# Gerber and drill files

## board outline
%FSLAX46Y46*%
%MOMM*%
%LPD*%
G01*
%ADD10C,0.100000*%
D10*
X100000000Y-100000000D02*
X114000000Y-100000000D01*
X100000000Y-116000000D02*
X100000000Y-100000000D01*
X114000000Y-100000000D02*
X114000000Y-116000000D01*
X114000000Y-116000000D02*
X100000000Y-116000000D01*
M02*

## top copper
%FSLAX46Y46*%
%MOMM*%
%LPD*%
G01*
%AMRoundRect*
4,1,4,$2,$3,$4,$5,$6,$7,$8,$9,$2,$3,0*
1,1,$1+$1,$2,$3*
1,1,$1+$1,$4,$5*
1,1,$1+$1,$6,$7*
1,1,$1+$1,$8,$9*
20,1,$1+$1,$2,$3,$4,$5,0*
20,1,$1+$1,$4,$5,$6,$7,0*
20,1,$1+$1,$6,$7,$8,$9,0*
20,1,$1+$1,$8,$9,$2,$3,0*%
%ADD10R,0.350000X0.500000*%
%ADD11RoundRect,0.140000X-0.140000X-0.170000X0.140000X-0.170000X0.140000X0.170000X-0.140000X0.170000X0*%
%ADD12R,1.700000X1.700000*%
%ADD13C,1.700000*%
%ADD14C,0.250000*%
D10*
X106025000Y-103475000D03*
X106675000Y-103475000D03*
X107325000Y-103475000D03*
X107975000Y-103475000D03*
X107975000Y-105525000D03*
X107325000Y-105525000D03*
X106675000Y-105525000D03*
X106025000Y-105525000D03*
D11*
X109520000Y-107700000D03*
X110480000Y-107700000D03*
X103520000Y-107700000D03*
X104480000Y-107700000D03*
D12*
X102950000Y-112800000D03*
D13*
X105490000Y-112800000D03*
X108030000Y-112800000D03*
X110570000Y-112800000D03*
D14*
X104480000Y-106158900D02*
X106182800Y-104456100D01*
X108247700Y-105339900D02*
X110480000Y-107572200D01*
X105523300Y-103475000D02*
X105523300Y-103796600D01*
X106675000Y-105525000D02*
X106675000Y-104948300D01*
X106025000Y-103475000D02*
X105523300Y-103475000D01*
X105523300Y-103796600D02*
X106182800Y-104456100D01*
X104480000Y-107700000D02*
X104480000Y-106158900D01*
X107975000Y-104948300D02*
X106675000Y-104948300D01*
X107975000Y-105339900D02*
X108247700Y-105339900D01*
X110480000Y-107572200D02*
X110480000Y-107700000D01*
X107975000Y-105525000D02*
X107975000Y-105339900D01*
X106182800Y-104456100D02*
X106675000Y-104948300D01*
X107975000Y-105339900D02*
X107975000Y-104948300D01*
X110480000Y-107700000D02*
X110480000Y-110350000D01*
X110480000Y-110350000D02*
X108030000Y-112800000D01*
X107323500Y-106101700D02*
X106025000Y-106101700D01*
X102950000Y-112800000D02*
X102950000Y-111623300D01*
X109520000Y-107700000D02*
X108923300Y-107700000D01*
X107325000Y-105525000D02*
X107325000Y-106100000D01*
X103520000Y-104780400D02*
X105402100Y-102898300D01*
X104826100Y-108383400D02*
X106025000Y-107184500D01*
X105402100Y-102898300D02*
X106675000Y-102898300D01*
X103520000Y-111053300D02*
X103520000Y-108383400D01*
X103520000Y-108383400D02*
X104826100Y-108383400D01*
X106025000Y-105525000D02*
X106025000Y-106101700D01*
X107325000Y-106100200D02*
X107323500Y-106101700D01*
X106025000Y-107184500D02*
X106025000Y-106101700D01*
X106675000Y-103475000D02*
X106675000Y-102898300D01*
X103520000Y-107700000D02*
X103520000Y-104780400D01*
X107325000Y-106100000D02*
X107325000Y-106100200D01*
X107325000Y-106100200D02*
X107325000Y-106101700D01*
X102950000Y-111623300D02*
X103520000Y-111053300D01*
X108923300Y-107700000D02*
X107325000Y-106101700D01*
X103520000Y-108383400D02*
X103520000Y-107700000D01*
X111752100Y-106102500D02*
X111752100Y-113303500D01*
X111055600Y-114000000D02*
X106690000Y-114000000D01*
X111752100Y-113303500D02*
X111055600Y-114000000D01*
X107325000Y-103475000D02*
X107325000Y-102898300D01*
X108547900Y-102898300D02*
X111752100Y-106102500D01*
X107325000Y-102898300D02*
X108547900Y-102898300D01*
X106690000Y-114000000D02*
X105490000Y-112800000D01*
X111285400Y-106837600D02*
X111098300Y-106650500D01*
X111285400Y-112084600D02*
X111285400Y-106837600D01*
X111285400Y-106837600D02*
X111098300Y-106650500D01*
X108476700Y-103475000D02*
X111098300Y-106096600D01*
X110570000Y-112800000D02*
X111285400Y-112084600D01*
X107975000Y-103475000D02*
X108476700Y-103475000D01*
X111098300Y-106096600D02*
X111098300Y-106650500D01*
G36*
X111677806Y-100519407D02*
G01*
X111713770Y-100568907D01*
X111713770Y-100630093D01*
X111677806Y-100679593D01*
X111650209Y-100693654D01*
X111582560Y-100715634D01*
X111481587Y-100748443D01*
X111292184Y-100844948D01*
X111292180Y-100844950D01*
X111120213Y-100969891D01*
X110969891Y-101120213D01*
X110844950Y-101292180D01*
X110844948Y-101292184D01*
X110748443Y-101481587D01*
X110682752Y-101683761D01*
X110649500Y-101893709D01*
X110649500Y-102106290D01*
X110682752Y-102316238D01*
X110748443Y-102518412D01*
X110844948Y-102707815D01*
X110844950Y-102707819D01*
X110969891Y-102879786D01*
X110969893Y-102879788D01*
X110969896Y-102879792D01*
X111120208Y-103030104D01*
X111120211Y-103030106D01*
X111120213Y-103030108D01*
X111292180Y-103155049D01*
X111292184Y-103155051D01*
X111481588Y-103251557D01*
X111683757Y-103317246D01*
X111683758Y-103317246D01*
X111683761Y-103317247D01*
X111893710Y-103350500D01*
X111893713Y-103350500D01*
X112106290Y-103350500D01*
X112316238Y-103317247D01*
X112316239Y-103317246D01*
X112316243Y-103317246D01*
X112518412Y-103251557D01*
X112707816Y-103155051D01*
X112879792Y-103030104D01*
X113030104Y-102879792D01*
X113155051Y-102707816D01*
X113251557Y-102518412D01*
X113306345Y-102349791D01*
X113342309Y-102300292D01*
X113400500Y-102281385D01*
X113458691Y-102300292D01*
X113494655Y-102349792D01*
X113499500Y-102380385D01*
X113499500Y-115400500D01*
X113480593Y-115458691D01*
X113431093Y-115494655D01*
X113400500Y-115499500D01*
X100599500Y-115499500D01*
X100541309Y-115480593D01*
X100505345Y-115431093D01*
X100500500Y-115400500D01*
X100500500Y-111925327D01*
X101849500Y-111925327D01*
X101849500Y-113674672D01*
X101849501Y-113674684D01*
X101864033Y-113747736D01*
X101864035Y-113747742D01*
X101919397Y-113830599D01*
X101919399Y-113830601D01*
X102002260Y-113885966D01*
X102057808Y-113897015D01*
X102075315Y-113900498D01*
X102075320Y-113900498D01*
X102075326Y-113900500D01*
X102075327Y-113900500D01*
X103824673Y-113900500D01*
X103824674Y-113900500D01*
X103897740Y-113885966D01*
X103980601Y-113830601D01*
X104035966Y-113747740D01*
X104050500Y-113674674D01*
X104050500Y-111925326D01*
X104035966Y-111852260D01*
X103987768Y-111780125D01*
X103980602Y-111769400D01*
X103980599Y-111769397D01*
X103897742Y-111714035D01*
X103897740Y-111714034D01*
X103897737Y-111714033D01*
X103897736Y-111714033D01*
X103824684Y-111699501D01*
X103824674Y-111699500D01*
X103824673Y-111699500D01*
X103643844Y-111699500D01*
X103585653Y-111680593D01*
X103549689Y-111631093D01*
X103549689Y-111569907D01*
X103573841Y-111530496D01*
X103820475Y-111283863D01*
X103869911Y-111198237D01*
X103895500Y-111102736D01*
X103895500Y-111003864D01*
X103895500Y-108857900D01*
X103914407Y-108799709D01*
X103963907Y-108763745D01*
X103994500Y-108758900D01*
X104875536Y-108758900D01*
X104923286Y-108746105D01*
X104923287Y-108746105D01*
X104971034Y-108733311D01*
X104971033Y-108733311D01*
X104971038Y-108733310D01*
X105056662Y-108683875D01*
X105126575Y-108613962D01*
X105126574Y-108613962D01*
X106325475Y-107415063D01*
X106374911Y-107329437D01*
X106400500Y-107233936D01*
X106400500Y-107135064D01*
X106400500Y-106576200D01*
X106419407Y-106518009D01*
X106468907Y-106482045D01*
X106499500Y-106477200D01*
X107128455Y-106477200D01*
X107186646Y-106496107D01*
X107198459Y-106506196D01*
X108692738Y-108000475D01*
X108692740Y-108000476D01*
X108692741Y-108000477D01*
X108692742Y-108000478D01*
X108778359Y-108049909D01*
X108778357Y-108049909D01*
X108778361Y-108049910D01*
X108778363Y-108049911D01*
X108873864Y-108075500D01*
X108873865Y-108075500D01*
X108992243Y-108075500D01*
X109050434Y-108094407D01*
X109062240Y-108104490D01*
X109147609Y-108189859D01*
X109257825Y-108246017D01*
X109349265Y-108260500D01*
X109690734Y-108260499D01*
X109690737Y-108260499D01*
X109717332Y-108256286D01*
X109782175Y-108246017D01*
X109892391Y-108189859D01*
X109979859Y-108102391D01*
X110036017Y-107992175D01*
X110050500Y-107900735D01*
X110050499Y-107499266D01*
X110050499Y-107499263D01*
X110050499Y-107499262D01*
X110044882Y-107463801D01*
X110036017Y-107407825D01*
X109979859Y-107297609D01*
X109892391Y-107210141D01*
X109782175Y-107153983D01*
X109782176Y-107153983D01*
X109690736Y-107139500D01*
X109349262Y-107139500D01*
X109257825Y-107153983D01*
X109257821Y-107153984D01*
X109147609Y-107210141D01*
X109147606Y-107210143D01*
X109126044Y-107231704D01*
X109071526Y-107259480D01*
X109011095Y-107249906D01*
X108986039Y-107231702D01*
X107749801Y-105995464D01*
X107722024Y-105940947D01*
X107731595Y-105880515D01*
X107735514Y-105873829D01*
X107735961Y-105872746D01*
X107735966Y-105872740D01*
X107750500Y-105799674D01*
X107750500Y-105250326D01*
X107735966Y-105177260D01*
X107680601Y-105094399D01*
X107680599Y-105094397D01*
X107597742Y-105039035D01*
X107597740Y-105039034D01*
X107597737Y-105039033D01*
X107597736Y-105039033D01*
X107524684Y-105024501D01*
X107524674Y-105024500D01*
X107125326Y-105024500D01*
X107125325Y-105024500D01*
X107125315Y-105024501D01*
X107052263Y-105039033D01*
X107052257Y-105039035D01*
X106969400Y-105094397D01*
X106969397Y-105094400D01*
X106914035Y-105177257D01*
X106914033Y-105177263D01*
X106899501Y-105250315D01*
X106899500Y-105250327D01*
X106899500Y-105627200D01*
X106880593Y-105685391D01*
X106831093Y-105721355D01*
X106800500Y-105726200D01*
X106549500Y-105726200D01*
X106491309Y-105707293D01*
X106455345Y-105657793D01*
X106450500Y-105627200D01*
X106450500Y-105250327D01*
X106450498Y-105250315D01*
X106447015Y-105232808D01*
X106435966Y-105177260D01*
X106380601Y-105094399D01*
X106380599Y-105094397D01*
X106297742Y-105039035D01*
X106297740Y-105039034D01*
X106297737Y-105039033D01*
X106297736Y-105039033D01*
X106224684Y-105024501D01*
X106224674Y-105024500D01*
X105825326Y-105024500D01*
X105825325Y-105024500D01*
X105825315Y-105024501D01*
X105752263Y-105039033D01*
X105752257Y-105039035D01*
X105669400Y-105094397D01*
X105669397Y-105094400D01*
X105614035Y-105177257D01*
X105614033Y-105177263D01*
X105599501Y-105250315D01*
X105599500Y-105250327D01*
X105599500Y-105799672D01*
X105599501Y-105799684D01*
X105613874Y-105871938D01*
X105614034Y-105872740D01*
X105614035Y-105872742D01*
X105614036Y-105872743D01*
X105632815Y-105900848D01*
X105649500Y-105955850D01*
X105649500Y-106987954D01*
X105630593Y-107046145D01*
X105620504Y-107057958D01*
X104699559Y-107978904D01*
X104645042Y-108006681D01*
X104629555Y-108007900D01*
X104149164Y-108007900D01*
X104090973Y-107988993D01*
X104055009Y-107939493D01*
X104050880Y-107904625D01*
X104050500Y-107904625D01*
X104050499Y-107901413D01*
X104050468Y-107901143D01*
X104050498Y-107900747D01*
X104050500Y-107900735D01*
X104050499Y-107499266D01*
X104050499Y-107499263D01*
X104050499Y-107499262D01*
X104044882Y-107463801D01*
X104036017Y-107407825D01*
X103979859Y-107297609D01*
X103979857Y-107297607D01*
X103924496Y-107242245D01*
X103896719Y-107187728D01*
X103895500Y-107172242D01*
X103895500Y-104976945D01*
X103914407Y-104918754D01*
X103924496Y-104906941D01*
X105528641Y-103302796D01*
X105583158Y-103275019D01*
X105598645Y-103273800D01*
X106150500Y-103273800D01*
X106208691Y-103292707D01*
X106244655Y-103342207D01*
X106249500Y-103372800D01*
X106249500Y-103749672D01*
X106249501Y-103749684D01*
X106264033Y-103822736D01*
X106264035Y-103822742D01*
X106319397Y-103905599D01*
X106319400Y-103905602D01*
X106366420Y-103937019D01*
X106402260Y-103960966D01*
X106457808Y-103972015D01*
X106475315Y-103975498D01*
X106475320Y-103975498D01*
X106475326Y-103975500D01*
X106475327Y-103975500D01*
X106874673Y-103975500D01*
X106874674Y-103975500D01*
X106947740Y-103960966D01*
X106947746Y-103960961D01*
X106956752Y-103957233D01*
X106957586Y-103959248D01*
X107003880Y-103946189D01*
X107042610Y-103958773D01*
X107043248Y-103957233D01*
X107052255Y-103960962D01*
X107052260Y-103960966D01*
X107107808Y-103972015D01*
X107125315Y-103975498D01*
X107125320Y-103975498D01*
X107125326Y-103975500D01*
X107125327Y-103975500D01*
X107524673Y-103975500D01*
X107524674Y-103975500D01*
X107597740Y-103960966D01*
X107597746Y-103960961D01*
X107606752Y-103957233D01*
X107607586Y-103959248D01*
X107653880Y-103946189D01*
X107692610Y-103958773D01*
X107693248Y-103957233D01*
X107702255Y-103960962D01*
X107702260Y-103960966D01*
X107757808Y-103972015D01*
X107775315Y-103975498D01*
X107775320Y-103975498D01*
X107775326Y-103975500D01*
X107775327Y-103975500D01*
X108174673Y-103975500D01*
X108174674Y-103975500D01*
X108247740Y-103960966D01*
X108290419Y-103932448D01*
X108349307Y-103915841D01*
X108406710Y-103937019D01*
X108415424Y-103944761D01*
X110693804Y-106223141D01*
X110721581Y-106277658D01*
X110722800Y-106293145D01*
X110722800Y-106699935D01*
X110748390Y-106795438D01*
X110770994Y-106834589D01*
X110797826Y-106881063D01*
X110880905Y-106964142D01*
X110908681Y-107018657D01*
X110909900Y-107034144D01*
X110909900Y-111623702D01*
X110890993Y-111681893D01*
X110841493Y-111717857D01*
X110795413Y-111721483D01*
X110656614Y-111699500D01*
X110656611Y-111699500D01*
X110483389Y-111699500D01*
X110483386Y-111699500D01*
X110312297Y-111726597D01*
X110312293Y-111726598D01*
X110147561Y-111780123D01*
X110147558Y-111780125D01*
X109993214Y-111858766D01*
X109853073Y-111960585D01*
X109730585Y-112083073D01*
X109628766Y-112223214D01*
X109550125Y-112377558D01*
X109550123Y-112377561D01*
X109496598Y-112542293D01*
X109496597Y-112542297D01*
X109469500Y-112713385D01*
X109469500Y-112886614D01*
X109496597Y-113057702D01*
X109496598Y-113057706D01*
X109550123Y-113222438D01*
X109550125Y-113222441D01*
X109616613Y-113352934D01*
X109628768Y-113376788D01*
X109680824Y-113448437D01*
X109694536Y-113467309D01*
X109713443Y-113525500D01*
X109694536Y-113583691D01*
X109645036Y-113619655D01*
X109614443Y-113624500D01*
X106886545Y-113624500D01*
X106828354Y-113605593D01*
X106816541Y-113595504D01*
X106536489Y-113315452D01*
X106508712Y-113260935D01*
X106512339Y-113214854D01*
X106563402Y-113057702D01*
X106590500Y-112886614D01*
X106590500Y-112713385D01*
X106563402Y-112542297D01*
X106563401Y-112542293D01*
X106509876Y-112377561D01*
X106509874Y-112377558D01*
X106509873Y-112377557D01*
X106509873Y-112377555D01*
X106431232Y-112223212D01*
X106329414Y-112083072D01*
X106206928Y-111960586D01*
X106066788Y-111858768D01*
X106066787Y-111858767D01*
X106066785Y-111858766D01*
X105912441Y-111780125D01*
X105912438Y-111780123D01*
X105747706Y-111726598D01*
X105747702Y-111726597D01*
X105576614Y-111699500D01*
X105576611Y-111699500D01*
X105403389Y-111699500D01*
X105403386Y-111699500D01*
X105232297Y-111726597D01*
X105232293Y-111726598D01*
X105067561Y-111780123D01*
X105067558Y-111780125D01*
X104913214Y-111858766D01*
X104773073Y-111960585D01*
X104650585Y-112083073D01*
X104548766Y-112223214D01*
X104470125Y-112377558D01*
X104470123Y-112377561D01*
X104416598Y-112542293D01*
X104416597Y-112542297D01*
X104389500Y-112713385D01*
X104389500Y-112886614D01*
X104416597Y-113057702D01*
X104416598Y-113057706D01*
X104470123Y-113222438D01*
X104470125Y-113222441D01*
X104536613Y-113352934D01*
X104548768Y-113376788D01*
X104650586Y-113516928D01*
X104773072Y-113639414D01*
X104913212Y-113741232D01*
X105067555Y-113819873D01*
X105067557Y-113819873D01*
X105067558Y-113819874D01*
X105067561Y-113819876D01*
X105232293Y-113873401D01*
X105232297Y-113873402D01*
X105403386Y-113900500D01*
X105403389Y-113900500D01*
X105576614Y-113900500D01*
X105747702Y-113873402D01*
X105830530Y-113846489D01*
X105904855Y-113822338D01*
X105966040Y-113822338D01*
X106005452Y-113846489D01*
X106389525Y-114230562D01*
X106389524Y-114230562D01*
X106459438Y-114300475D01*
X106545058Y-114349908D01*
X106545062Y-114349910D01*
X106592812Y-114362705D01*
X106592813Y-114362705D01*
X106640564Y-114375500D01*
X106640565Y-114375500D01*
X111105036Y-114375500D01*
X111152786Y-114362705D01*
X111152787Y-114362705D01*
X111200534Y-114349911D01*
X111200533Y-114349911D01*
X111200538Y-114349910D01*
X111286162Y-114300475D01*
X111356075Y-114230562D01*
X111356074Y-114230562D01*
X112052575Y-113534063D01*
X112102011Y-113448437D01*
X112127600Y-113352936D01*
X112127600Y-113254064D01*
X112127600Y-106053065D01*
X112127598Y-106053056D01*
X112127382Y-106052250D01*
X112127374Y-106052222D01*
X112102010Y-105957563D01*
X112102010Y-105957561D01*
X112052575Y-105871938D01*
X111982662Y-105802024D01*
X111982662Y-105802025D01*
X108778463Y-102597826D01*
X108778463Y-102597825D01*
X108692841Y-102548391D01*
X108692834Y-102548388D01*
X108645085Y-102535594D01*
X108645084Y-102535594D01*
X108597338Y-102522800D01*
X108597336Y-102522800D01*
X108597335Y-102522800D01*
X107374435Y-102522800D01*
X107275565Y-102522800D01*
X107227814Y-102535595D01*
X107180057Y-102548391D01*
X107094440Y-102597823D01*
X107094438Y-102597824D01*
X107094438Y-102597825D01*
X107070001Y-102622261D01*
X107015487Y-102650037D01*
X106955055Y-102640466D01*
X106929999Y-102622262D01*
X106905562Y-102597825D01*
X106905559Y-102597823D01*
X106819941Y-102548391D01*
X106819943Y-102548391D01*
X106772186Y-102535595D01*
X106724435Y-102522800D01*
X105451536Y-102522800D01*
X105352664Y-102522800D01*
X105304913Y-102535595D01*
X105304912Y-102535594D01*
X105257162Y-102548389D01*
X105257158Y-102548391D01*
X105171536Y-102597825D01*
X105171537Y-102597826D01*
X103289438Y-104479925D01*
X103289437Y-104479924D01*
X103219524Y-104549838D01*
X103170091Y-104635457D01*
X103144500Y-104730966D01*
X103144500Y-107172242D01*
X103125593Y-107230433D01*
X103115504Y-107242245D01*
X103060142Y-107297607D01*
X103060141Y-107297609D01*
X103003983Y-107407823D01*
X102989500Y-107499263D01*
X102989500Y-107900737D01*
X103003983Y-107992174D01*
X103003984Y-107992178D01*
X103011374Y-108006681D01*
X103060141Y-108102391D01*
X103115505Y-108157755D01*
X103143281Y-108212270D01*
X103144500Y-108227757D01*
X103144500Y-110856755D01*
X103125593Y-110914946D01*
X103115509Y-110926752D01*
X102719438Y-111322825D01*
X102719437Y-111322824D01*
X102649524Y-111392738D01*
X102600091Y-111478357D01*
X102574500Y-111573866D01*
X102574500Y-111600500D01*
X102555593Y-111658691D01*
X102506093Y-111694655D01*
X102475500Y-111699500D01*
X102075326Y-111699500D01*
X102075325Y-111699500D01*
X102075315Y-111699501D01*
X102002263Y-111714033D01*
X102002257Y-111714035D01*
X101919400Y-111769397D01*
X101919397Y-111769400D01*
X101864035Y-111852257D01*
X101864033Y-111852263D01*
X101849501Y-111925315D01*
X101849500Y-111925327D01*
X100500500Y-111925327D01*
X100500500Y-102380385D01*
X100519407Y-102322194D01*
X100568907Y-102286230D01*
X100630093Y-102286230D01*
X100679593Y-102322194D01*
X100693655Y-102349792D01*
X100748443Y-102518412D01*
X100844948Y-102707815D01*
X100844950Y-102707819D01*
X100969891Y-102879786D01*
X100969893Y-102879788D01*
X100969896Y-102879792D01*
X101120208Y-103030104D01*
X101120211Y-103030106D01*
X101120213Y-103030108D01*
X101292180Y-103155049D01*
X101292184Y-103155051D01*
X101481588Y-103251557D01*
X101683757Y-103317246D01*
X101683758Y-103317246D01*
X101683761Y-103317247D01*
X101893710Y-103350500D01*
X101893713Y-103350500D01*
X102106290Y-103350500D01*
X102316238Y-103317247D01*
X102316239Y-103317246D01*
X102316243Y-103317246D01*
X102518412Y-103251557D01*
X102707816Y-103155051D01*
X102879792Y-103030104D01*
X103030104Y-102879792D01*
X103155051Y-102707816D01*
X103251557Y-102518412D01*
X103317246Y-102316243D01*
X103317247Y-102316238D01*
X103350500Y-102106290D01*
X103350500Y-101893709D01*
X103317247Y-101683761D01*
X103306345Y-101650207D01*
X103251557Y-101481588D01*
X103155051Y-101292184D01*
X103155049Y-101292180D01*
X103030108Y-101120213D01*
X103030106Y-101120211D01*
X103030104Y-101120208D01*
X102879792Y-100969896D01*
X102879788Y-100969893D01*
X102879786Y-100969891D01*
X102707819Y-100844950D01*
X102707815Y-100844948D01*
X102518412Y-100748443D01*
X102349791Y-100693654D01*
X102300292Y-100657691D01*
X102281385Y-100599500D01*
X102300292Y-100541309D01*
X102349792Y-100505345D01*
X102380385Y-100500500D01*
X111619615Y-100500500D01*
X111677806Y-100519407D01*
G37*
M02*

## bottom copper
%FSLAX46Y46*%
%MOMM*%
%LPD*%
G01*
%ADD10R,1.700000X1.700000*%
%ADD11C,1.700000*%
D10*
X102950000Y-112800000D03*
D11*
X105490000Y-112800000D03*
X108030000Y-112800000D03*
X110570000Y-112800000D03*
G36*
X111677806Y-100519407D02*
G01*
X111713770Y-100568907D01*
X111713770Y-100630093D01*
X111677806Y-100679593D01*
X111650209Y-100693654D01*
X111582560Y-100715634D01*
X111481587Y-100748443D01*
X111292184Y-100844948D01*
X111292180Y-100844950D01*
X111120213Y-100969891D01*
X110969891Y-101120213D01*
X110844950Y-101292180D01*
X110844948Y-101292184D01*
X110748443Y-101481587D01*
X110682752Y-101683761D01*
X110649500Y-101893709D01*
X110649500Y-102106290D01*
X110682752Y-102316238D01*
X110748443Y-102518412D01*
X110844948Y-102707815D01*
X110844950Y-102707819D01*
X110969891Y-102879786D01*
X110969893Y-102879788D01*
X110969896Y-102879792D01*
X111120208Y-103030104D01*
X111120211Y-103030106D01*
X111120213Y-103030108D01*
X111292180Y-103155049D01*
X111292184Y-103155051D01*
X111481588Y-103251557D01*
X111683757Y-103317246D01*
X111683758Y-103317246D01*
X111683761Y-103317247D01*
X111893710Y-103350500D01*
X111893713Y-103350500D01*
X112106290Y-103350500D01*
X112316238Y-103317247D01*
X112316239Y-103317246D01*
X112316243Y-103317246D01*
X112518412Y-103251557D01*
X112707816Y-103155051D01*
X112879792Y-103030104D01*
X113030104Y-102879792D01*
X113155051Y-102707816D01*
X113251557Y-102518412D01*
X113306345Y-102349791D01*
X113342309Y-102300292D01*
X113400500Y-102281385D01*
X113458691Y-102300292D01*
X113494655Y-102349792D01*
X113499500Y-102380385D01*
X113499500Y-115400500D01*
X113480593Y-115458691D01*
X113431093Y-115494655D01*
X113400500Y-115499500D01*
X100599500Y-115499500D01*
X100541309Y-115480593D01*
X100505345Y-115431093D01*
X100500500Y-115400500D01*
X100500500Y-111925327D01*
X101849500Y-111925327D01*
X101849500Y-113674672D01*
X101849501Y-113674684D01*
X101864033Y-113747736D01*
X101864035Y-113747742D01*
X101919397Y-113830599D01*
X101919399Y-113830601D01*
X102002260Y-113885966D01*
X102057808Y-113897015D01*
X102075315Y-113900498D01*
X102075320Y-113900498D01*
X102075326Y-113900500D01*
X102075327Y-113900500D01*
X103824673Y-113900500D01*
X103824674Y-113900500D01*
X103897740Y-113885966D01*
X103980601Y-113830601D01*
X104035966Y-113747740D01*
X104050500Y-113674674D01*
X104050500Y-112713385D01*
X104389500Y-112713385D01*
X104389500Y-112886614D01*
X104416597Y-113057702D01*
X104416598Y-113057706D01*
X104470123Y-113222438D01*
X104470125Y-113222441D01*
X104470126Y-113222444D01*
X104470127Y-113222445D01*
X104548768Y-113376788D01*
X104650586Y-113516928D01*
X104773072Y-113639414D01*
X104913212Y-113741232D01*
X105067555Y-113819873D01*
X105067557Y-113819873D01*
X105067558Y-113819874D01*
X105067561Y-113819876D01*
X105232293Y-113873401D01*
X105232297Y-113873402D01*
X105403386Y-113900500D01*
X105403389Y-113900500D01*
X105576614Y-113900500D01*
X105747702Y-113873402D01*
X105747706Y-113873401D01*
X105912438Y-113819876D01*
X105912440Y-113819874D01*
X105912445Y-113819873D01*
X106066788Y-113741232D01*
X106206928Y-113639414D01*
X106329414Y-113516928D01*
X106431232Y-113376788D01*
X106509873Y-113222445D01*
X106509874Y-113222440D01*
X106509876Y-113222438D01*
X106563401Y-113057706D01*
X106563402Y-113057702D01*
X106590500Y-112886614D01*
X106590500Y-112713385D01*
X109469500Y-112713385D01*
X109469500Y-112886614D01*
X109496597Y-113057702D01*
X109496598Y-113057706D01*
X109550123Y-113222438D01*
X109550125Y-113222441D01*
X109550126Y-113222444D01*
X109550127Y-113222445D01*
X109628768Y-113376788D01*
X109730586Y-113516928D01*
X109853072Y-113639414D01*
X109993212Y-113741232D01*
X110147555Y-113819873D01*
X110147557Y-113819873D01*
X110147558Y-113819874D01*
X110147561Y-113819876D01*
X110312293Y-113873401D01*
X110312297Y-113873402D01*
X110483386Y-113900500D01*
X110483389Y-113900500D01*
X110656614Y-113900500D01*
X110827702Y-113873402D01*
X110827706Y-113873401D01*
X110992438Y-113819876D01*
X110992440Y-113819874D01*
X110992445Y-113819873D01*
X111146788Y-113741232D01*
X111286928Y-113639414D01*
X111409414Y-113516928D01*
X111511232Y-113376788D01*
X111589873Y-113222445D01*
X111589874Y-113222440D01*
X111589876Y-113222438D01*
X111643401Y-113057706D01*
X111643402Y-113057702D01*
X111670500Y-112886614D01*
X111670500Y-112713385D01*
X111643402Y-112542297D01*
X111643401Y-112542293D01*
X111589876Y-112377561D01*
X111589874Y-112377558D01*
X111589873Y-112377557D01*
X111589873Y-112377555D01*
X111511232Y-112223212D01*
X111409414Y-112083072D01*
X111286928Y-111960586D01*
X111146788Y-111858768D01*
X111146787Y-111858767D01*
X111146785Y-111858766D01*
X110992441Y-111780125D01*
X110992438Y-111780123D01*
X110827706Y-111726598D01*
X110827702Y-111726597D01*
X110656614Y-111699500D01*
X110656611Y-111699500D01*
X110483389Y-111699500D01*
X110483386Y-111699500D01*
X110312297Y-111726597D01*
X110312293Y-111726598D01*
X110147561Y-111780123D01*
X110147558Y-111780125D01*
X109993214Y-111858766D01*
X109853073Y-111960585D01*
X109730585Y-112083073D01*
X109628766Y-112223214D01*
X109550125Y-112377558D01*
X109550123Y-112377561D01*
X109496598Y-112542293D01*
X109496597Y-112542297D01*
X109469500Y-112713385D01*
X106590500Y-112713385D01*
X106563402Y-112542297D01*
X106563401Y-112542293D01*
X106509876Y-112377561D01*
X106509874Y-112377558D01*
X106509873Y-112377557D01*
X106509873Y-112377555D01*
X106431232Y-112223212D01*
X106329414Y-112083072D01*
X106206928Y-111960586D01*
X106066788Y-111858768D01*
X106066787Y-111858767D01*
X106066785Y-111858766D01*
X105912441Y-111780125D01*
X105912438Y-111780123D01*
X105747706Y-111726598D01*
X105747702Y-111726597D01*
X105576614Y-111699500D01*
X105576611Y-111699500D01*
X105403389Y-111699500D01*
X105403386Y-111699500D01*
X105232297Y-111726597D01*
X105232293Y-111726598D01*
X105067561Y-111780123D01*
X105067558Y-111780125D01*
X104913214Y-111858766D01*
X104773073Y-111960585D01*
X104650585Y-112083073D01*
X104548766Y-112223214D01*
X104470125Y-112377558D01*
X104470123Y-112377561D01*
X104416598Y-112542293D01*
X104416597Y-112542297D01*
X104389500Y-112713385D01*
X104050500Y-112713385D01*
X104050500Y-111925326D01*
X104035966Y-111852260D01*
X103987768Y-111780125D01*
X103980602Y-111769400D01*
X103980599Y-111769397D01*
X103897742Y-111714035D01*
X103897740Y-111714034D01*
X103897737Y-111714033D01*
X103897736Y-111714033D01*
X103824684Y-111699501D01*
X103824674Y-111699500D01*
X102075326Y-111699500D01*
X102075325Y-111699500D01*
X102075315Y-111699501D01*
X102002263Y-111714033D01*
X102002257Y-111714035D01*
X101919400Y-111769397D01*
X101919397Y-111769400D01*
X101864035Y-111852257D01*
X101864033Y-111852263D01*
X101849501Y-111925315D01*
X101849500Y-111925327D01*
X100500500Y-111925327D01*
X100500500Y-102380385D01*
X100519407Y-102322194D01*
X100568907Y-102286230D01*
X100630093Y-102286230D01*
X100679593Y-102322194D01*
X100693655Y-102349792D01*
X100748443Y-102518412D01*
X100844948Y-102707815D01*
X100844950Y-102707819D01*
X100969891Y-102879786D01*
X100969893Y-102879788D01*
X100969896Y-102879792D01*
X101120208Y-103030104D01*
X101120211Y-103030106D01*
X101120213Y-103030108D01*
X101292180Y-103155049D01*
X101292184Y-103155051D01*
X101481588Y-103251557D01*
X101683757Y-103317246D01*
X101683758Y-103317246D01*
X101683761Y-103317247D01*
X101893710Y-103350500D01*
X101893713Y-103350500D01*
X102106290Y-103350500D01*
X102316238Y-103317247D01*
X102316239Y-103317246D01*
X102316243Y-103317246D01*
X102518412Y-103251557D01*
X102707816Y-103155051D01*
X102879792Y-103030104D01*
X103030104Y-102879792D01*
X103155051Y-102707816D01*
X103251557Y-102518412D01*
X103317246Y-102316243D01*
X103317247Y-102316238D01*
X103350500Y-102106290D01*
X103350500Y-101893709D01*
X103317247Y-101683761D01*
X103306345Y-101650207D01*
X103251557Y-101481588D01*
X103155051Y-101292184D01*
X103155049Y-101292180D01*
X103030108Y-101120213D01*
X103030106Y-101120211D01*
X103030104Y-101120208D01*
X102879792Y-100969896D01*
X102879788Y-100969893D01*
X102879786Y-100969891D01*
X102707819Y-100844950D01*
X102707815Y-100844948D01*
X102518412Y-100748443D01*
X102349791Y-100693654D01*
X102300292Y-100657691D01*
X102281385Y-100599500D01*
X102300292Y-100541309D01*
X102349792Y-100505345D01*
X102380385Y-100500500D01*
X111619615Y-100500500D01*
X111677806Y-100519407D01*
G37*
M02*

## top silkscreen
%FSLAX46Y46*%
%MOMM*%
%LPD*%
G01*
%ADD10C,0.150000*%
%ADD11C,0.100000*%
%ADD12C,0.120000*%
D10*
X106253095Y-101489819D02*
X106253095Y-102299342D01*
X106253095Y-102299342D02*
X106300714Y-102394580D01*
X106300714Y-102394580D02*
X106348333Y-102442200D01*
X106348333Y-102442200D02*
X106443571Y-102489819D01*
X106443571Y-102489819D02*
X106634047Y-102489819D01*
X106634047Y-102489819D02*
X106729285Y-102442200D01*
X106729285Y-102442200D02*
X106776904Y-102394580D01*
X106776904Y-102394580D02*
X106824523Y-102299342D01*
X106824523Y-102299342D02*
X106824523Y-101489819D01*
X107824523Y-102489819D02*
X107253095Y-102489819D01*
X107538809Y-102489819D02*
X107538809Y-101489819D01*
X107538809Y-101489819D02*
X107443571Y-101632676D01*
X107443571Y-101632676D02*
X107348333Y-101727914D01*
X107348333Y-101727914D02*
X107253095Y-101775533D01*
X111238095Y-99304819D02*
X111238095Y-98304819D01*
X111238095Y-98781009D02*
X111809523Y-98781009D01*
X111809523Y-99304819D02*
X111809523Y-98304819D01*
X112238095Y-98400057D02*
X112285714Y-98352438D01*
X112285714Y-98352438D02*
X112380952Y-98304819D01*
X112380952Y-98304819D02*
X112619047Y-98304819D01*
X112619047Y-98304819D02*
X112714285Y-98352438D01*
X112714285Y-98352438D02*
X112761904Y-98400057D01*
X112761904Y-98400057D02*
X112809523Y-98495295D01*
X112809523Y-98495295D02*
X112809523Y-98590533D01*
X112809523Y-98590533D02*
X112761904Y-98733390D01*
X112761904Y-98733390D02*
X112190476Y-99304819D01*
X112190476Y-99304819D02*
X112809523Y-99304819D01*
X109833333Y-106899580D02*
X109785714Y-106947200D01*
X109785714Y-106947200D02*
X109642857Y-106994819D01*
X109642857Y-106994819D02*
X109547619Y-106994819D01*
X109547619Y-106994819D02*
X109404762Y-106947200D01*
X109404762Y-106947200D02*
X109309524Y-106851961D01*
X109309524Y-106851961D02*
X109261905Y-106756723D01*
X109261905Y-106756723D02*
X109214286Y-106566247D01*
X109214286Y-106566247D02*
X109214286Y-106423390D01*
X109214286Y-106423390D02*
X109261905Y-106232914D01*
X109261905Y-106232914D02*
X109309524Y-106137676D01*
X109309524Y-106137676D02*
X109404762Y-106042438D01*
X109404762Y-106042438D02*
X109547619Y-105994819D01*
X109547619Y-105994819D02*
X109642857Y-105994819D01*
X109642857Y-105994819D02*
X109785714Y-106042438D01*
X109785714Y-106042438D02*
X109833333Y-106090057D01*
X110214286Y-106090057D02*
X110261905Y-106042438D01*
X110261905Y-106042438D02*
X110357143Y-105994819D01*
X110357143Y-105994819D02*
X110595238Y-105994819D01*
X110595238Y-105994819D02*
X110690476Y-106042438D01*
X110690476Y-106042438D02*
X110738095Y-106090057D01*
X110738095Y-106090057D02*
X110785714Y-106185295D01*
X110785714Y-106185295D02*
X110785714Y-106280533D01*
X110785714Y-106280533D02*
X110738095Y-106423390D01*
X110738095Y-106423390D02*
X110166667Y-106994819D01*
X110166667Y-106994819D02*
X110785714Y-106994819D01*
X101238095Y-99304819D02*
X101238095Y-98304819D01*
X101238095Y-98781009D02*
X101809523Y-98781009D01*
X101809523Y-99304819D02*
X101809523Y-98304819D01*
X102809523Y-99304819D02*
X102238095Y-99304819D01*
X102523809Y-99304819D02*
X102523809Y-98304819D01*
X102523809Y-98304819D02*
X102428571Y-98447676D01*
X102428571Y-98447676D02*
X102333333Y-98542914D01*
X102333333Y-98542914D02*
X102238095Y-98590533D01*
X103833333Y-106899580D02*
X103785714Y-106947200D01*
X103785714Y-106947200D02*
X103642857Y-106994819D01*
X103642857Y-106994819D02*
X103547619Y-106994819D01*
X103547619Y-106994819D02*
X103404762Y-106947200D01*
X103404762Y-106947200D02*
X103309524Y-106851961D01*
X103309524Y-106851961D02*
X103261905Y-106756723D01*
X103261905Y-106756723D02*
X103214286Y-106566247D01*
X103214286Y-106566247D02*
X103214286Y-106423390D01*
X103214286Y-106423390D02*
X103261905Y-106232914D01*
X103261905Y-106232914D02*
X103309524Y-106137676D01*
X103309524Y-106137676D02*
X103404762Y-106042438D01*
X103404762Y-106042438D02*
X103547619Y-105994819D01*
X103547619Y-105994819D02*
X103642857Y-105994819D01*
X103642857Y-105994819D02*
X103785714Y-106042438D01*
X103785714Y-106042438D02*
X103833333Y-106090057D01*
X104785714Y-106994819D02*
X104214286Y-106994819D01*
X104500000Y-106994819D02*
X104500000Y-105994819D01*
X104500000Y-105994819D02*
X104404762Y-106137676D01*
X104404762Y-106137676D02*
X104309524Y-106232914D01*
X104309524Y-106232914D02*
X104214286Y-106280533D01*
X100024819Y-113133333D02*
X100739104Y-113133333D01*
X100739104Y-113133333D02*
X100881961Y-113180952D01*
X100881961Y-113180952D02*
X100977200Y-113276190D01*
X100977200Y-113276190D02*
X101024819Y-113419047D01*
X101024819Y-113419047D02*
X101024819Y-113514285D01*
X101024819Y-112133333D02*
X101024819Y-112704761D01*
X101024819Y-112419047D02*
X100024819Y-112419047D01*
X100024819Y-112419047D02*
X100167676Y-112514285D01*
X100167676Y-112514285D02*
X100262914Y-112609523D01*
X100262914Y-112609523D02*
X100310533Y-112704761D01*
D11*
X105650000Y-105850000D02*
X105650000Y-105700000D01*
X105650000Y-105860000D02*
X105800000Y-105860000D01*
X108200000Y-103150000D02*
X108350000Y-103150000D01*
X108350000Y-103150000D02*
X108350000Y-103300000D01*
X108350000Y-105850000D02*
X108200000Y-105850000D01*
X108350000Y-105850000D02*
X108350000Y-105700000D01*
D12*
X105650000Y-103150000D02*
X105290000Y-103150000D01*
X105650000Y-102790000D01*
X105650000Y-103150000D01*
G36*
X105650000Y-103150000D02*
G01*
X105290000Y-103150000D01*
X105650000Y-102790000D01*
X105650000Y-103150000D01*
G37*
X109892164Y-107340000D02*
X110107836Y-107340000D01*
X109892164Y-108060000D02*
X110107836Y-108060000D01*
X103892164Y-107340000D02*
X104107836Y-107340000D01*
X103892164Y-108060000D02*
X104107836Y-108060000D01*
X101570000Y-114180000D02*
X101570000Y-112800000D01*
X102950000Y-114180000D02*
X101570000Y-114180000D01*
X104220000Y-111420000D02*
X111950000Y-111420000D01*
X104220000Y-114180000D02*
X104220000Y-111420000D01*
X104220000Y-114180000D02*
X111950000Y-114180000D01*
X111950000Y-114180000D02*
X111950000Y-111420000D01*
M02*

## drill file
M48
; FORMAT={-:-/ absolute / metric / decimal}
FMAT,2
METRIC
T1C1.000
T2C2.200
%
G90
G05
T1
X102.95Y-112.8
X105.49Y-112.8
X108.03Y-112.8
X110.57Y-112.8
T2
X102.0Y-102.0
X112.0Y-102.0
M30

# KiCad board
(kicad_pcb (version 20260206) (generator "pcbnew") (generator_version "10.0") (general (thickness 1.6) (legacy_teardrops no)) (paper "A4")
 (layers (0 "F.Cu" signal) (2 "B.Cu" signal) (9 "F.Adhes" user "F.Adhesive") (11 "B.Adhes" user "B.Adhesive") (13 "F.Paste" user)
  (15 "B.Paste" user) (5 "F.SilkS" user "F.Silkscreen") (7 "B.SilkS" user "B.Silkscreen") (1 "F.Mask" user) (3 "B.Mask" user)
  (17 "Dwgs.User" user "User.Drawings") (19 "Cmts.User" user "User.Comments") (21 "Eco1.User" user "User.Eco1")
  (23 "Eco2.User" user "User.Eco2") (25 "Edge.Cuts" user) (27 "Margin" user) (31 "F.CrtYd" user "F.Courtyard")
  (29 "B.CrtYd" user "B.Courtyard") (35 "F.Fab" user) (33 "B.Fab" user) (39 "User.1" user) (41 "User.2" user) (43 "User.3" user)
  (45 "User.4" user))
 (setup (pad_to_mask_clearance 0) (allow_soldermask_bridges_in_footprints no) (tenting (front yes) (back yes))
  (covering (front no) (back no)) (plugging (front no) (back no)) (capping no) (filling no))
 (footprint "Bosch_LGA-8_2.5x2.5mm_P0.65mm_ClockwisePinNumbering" (layer "F.Cu") (at 107 104.5)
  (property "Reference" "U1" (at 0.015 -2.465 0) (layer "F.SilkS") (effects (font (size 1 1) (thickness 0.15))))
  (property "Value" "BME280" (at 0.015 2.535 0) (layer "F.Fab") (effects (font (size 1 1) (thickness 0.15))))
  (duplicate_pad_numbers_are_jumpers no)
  (fp_line (start -1.35 1.35) (end -1.35 1.2) (stroke (width 0.1) (type solid)) (layer "F.SilkS"))
  (fp_line (start -1.35 1.36) (end -1.2 1.36) (stroke (width 0.1) (type solid)) (layer "F.SilkS"))
  (fp_line (start 1.2 -1.35) (end 1.35 -1.35) (stroke (width 0.1) (type solid)) (layer "F.SilkS"))
  (fp_line (start 1.35 -1.35) (end 1.35 -1.2) (stroke (width 0.1) (type solid)) (layer "F.SilkS"))
  (fp_line (start 1.35 1.35) (end 1.2 1.35) (stroke (width 0.1) (type solid)) (layer "F.SilkS"))
  (fp_line (start 1.35 1.35) (end 1.35 1.2) (stroke (width 0.1) (type solid)) (layer "F.SilkS"))
  (fp_poly
   (pts (xy -1.35 -1.35) (xy -1.71 -1.35) (xy -1.35 -1.71) (xy -1.35 -1.35)) (stroke (width 0.12) (type solid)) (fill yes) (layer "F.SilkS"))
  (pad "1" smd rect (at -0.975 -1.025 90) (size 0.5 0.35) (layers "F.Cu" "F.Mask" "F.Paste") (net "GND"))
  (pad "2" smd rect (at -0.325 -1.025 90) (size 0.5 0.35) (layers "F.Cu" "F.Mask" "F.Paste") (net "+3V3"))
  (pad "3" smd rect (at 0.325 -1.025 90) (size 0.5 0.35) (layers "F.Cu" "F.Mask" "F.Paste") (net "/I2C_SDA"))
  (pad "4" smd rect (at 0.975 -1.025 90) (size 0.5 0.35) (layers "F.Cu" "F.Mask" "F.Paste") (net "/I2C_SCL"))
  (pad "5" smd rect (at 0.975 1.025 90) (size 0.5 0.35) (layers "F.Cu" "F.Mask" "F.Paste") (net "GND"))
  (pad "6" smd rect (at 0.325 1.025 90) (size 0.5 0.35) (layers "F.Cu" "F.Mask" "F.Paste") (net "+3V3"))
  (pad "7" smd rect (at -0.325 1.025 90) (size 0.5 0.35) (layers "F.Cu" "F.Mask" "F.Paste") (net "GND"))
  (pad "8" smd rect (at -0.975 1.025 90) (size 0.5 0.35) (layers "F.Cu" "F.Mask" "F.Paste") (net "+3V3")))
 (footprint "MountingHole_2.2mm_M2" (layer "F.Cu") (at 112 102)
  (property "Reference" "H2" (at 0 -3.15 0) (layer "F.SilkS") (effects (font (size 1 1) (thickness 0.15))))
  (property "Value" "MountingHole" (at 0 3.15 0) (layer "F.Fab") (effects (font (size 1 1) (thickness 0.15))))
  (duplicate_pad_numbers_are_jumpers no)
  (pad "" np_thru_hole circle (at 0 0) (size 2.2 2.2) (drill 2.2) (layers "*.Cu" "*.Mask")))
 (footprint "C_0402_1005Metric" (layer "F.Cu") (at 110 107.7)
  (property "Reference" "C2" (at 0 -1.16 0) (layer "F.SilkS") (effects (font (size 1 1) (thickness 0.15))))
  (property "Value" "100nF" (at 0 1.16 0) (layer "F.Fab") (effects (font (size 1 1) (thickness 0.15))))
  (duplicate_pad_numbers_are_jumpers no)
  (fp_line (start -0.107836 -0.36) (end 0.107836 -0.36) (stroke (width 0.12) (type solid)) (layer "F.SilkS"))
  (fp_line (start -0.107836 0.36) (end 0.107836 0.36) (stroke (width 0.12) (type solid)) (layer "F.SilkS"))
  (pad "1" smd roundrect (at -0.48 0) (size 0.56 0.62) (layers "F.Cu" "F.Mask" "F.Paste") (roundrect_rratio 0.25) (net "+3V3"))
  (pad "2" smd roundrect (at 0.48 0) (size 0.56 0.62) (layers "F.Cu" "F.Mask" "F.Paste") (roundrect_rratio 0.25) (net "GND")))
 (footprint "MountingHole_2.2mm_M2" (layer "F.Cu") (at 102 102)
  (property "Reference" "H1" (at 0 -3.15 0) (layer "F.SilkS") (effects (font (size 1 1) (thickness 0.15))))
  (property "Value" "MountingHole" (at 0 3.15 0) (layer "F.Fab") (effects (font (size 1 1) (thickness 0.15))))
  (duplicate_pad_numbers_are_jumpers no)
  (pad "" np_thru_hole circle (at 0 0) (size 2.2 2.2) (drill 2.2) (layers "*.Cu" "*.Mask")))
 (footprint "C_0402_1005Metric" (layer "F.Cu") (at 104 107.7)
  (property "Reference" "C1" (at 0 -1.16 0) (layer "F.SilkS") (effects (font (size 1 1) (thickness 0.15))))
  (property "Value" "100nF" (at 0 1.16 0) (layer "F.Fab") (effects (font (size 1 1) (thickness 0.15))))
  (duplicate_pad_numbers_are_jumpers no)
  (fp_line (start -0.107836 -0.36) (end 0.107836 -0.36) (stroke (width 0.12) (type solid)) (layer "F.SilkS"))
  (fp_line (start -0.107836 0.36) (end 0.107836 0.36) (stroke (width 0.12) (type solid)) (layer "F.SilkS"))
  (pad "1" smd roundrect (at -0.48 0) (size 0.56 0.62) (layers "F.Cu" "F.Mask" "F.Paste") (roundrect_rratio 0.25) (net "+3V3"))
  (pad "2" smd roundrect (at 0.48 0) (size 0.56 0.62) (layers "F.Cu" "F.Mask" "F.Paste") (roundrect_rratio 0.25) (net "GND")))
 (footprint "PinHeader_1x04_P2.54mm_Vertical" (layer "F.Cu") (at 102.95 112.8 90)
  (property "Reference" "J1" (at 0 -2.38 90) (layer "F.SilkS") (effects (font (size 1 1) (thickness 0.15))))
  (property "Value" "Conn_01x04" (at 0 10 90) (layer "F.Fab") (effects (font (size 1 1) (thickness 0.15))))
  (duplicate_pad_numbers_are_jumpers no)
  (fp_line (start -1.38 -1.38) (end 0 -1.38) (stroke (width 0.12) (type solid)) (layer "F.SilkS"))
  (fp_line (start -1.38 0) (end -1.38 -1.38) (stroke (width 0.12) (type solid)) (layer "F.SilkS"))
  (fp_line (start 1.38 1.27) (end 1.38 9) (stroke (width 0.12) (type solid)) (layer "F.SilkS"))
  (fp_line (start -1.38 1.27) (end 1.38 1.27) (stroke (width 0.12) (type solid)) (layer "F.SilkS"))
  (fp_line (start -1.38 1.27) (end -1.38 9) (stroke (width 0.12) (type solid)) (layer "F.SilkS"))
  (fp_line (start -1.38 9) (end 1.38 9) (stroke (width 0.12) (type solid)) (layer "F.SilkS"))
  (pad "1" thru_hole rect (at 0 0 90) (size 1.7 1.7) (drill 1) (layers "*.Cu" "*.Mask") (remove_unused_layers no) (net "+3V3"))
  (pad "2" thru_hole circle (at 0 2.54 90) (size 1.7 1.7) (drill 1) (layers "*.Cu" "*.Mask") (remove_unused_layers no) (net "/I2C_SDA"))
  (pad "3" thru_hole circle (at 0 5.08 90) (size 1.7 1.7) (drill 1) (layers "*.Cu" "*.Mask") (remove_unused_layers no) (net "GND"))
  (pad "4" thru_hole circle (at 0 7.62 90) (size 1.7 1.7) (drill 1) (layers "*.Cu" "*.Mask") (remove_unused_layers no) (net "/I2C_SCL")))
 (gr_line (start 100 100) (end 114 100) (stroke (width 0.1) (type default)) (layer "Edge.Cuts"))
 (gr_line (start 100 116) (end 100 100) (stroke (width 0.1) (type default)) (layer "Edge.Cuts"))
 (gr_line (start 114 100) (end 114 116) (stroke (width 0.1) (type default)) (layer "Edge.Cuts"))
 (gr_line (start 114 116) (end 100 116) (stroke (width 0.1) (type default)) (layer "Edge.Cuts"))
 (segment (start 104.48 106.1589) (end 106.1828 104.4561) (width 0.25) (layer "F.Cu") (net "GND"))
 (segment (start 108.2477 105.3399) (end 110.48 107.5722) (width 0.25) (layer "F.Cu") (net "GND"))
 (segment (start 105.5233 103.475) (end 105.5233 103.7966) (width 0.25) (layer "F.Cu") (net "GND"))
 (segment (start 106.675 105.525) (end 106.675 104.9483) (width 0.25) (layer "F.Cu") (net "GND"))
 (segment (start 106.025 103.475) (end 105.5233 103.475) (width 0.25) (layer "F.Cu") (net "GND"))
 (segment (start 105.5233 103.7966) (end 106.1828 104.4561) (width 0.25) (layer "F.Cu") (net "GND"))
 (segment (start 104.48 107.7) (end 104.48 106.1589) (width 0.25) (layer "F.Cu") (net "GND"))
 (segment (start 107.975 104.9483) (end 106.675 104.9483) (width 0.25) (layer "F.Cu") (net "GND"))
 (segment (start 107.975 105.3399) (end 108.2477 105.3399) (width 0.25) (layer "F.Cu") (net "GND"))
 (segment (start 110.48 107.5722) (end 110.48 107.7) (width 0.25) (layer "F.Cu") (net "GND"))
 (segment (start 107.975 105.525) (end 107.975 105.3399) (width 0.25) (layer "F.Cu") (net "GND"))
 (segment (start 106.1828 104.4561) (end 106.675 104.9483) (width 0.25) (layer "F.Cu") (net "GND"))
 (segment (start 107.975 105.3399) (end 107.975 104.9483) (width 0.25) (layer "F.Cu") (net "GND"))
 (segment (start 110.48 107.7) (end 110.48 110.35) (width 0.25) (layer "F.Cu") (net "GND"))
 (segment (start 110.48 110.35) (end 108.03 112.8) (width 0.25) (layer "F.Cu") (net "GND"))
 (segment (start 107.3235 106.1017) (end 106.025 106.1017) (width 0.25) (layer "F.Cu") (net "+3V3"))
 (segment (start 102.95 112.8) (end 102.95 111.6233) (width 0.25) (layer "F.Cu") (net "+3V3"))
 (segment (start 109.52 107.7) (end 108.9233 107.7) (width 0.25) (layer "F.Cu") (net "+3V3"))
 (segment (start 107.325 105.525) (end 107.325 106.1) (width 0.25) (layer "F.Cu") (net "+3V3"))
 (segment (start 103.52 104.7804) (end 105.4021 102.8983) (width 0.25) (layer "F.Cu") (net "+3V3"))
 (segment (start 104.8261 108.3834) (end 106.025 107.1845) (width 0.25) (layer "F.Cu") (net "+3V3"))
 (segment (start 105.4021 102.8983) (end 106.675 102.8983) (width 0.25) (layer "F.Cu") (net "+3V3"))
 (segment (start 103.52 111.0533) (end 103.52 108.3834) (width 0.25) (layer "F.Cu") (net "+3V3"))
 (segment (start 103.52 108.3834) (end 104.8261 108.3834) (width 0.25) (layer "F.Cu") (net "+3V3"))
 (segment (start 106.025 105.525) (end 106.025 106.1017) (width 0.25) (layer "F.Cu") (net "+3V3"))
 (segment (start 107.325 106.1002) (end 107.3235 106.1017) (width 0.25) (layer "F.Cu") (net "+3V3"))
 (segment (start 106.025 107.1845) (end 106.025 106.1017) (width 0.25) (layer "F.Cu") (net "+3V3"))
 (segment (start 106.675 103.475) (end 106.675 102.8983) (width 0.25) (layer "F.Cu") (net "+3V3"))
 (segment (start 103.52 107.7) (end 103.52 104.7804) (width 0.25) (layer "F.Cu") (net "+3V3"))
 (segment (start 107.325 106.1) (end 107.325 106.1002) (width 0.25) (layer "F.Cu") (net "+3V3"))
 (segment (start 107.325 106.1002) (end 107.325 106.1017) (width 0.25) (layer "F.Cu") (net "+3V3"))
 (segment (start 102.95 111.6233) (end 103.52 111.0533) (width 0.25) (layer "F.Cu") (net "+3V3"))
 (segment (start 108.9233 107.7) (end 107.325 106.1017) (width 0.25) (layer "F.Cu") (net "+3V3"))
 (segment (start 103.52 108.3834) (end 103.52 107.7) (width 0.25) (layer "F.Cu") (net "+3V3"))
 (segment (start 111.7521 106.1025) (end 111.7521 113.3035) (width 0.25) (layer "F.Cu") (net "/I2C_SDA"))
 (segment (start 111.0556 114) (end 106.69 114) (width 0.25) (layer "F.Cu") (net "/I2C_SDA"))
 (segment (start 111.7521 113.3035) (end 111.0556 114) (width 0.25) (layer "F.Cu") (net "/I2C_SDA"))
 (segment (start 107.325 103.475) (end 107.325 102.8983) (width 0.25) (layer "F.Cu") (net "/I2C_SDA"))
 (segment (start 108.5479 102.8983) (end 111.7521 106.1025) (width 0.25) (layer "F.Cu") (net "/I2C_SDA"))
 (segment (start 107.325 102.8983) (end 108.5479 102.8983) (width 0.25) (layer "F.Cu") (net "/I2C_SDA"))
 (segment (start 106.69 114) (end 105.49 112.8) (width 0.25) (layer "F.Cu") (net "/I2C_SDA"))
 (segment (start 111.2854 106.8376) (end 111.0983 106.6505) (width 0.25) (layer "F.Cu") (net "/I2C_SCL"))
 (segment (start 111.2854 112.0846) (end 111.2854 106.8376) (width 0.25) (layer "F.Cu") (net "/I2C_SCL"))
 (segment (start 111.2854 106.8376) (end 111.0983 106.6505) (width 0.25) (layer "F.Cu") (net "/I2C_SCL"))
 (segment (start 108.4767 103.475) (end 111.0983 106.0966) (width 0.25) (layer "F.Cu") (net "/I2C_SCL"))
 (segment (start 110.57 112.8) (end 111.2854 112.0846) (width 0.25) (layer "F.Cu") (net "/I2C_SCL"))
 (segment (start 107.975 103.475) (end 108.4767 103.475) (width 0.25) (layer "F.Cu") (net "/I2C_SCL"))
 (segment (start 111.0983 106.0966) (end 111.0983 106.6505) (width 0.25) (layer "F.Cu") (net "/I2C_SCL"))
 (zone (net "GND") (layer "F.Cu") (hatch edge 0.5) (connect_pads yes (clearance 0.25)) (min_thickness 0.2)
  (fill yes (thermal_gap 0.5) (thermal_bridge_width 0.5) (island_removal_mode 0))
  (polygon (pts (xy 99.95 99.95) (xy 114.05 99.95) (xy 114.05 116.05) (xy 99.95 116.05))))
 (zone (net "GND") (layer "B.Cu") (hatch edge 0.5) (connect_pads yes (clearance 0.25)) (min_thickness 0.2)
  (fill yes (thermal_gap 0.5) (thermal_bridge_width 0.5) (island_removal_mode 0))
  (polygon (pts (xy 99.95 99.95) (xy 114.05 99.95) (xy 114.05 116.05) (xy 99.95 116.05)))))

